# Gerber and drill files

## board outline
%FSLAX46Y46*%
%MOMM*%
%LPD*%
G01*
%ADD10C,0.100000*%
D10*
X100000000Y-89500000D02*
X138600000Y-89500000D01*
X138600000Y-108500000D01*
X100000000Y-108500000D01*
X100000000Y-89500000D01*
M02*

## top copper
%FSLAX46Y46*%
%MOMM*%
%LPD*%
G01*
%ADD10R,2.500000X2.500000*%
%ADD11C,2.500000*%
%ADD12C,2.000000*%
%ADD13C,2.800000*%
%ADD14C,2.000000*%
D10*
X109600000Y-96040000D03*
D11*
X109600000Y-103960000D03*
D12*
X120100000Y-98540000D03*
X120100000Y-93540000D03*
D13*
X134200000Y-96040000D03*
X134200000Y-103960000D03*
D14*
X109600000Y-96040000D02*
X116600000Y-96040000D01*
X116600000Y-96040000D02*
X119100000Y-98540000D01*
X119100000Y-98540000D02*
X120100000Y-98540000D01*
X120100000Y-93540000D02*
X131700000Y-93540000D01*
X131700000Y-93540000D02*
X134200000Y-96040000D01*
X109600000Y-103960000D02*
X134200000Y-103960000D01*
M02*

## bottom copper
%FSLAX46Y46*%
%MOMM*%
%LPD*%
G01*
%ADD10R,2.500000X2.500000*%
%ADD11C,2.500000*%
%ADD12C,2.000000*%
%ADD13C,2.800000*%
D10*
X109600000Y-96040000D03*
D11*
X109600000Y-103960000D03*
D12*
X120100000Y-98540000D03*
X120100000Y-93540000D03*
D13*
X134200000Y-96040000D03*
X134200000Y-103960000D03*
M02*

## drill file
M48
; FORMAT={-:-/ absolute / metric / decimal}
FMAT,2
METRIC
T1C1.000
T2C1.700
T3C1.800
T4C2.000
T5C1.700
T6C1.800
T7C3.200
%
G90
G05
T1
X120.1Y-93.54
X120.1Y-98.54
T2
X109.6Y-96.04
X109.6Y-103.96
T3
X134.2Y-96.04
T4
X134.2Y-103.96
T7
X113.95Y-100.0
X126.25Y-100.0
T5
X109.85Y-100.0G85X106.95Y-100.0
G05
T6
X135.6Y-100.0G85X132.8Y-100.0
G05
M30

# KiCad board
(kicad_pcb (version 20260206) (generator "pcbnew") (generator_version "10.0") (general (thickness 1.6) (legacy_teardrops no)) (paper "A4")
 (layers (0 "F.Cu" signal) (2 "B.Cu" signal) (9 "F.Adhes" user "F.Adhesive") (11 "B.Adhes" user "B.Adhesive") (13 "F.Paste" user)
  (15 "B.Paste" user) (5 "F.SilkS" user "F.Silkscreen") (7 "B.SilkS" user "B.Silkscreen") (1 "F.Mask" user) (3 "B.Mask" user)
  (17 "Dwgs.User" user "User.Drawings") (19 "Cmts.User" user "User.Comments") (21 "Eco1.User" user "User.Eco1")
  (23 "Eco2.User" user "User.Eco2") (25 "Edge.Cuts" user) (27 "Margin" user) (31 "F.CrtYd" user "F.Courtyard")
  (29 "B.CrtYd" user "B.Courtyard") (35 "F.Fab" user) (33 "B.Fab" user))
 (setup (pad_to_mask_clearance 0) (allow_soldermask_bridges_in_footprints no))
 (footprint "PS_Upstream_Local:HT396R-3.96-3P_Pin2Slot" (layer "F.Cu") (at 109.6 100.0 270)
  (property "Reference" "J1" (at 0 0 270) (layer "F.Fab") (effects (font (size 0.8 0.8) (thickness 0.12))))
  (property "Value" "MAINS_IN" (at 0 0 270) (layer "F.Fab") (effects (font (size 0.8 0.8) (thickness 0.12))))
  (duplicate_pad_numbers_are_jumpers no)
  (pad "" np_thru_hole oval (at 0 1.2 270) (size 1.7 4.6) (drill oval 1.7 4.6) (layers "*.Cu" "*.Mask"))
  (pad "1" thru_hole rect (at -3.96 0 270) (size 2.5 2.5) (drill 1.700022) (layers "*.Cu" "*.Mask") (remove_unused_layers no) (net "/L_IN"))
  (pad "3" thru_hole circle (at 3.96 0 270) (size 2.5 2.5) (drill 1.700022) (layers "*.Cu" "*.Mask") (remove_unused_layers no) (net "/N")))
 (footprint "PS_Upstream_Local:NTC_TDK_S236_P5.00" (layer "F.Cu") (at 120.1 96.04 90)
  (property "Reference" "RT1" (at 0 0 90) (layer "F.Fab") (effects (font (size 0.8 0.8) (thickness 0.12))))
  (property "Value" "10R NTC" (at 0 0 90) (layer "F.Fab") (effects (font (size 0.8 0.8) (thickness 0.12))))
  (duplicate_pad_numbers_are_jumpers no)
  (pad "1" thru_hole circle (at -2.5 0 90) (size 2 2) (drill 1) (layers "*.Cu" "*.Mask") (remove_unused_layers no) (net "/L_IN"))
  (pad "2" thru_hole circle (at 2.5 0 90) (size 2 2) (drill 1) (layers "*.Cu" "*.Mask") (remove_unused_layers no) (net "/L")))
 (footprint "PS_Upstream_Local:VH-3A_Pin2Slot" (layer "F.Cu") (at 134.2 100.0 270)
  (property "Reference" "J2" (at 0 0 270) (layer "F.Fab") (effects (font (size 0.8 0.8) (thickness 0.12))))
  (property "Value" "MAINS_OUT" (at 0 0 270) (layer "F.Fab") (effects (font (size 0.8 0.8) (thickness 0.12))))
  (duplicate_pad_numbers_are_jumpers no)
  (pad "" np_thru_hole oval (at 0 0 270) (size 1.8 4.6) (drill oval 1.8 4.6) (layers "*.Cu" "*.Mask"))
  (pad "1" thru_hole circle (at -3.96 0 270) (size 2.8 2.8) (drill 1.799996) (layers "*.Cu" "*.Mask") (remove_unused_layers no) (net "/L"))
  (pad "3" thru_hole circle (at 3.96 0 270) (size 2.8 2.8) (drill 1.999996) (layers "*.Cu" "*.Mask") (remove_unused_layers no) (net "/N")))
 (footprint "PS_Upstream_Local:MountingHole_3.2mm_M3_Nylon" (layer "F.Cu") (at 113.95 100.0 0)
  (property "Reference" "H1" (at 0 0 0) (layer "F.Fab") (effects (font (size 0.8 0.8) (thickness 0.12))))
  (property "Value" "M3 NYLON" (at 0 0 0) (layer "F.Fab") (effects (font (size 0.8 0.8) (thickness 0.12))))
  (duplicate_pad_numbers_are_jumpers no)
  (pad "" np_thru_hole circle (at 0 0 0) (size 3.2 3.2) (drill 3.2) (layers "*.Cu" "*.Mask")))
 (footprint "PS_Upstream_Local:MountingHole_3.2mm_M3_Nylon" (layer "F.Cu") (at 126.25 100.0 0)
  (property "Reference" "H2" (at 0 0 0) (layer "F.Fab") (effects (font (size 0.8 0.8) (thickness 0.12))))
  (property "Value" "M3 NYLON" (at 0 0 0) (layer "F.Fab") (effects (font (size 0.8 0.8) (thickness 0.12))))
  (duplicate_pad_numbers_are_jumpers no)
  (pad "" np_thru_hole circle (at 0 0 0) (size 3.2 3.2) (drill 3.2) (layers "*.Cu" "*.Mask")))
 (gr_rect (start 100.0 89.5) (end 138.6 108.5) (stroke (width 0.1) (type solid)) (fill no) (layer "Edge.Cuts"))
 (segment (start 109.6 96.04) (end 116.6 96.04) (width 2.0) (layer "F.Cu") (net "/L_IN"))
 (segment (start 116.6 96.04) (end 119.1 98.54) (width 2.0) (layer "F.Cu") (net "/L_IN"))
 (segment (start 119.1 98.54) (end 120.1 98.54) (width 2.0) (layer "F.Cu") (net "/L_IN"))
 (segment (start 120.1 93.54) (end 131.7 93.54) (width 2.0) (layer "F.Cu") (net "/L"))
 (segment (start 131.7 93.54) (end 134.2 96.04) (width 2.0) (layer "F.Cu") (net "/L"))
 (segment (start 109.6 103.96) (end 134.2 103.96) (width 2.0) (layer "F.Cu") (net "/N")))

